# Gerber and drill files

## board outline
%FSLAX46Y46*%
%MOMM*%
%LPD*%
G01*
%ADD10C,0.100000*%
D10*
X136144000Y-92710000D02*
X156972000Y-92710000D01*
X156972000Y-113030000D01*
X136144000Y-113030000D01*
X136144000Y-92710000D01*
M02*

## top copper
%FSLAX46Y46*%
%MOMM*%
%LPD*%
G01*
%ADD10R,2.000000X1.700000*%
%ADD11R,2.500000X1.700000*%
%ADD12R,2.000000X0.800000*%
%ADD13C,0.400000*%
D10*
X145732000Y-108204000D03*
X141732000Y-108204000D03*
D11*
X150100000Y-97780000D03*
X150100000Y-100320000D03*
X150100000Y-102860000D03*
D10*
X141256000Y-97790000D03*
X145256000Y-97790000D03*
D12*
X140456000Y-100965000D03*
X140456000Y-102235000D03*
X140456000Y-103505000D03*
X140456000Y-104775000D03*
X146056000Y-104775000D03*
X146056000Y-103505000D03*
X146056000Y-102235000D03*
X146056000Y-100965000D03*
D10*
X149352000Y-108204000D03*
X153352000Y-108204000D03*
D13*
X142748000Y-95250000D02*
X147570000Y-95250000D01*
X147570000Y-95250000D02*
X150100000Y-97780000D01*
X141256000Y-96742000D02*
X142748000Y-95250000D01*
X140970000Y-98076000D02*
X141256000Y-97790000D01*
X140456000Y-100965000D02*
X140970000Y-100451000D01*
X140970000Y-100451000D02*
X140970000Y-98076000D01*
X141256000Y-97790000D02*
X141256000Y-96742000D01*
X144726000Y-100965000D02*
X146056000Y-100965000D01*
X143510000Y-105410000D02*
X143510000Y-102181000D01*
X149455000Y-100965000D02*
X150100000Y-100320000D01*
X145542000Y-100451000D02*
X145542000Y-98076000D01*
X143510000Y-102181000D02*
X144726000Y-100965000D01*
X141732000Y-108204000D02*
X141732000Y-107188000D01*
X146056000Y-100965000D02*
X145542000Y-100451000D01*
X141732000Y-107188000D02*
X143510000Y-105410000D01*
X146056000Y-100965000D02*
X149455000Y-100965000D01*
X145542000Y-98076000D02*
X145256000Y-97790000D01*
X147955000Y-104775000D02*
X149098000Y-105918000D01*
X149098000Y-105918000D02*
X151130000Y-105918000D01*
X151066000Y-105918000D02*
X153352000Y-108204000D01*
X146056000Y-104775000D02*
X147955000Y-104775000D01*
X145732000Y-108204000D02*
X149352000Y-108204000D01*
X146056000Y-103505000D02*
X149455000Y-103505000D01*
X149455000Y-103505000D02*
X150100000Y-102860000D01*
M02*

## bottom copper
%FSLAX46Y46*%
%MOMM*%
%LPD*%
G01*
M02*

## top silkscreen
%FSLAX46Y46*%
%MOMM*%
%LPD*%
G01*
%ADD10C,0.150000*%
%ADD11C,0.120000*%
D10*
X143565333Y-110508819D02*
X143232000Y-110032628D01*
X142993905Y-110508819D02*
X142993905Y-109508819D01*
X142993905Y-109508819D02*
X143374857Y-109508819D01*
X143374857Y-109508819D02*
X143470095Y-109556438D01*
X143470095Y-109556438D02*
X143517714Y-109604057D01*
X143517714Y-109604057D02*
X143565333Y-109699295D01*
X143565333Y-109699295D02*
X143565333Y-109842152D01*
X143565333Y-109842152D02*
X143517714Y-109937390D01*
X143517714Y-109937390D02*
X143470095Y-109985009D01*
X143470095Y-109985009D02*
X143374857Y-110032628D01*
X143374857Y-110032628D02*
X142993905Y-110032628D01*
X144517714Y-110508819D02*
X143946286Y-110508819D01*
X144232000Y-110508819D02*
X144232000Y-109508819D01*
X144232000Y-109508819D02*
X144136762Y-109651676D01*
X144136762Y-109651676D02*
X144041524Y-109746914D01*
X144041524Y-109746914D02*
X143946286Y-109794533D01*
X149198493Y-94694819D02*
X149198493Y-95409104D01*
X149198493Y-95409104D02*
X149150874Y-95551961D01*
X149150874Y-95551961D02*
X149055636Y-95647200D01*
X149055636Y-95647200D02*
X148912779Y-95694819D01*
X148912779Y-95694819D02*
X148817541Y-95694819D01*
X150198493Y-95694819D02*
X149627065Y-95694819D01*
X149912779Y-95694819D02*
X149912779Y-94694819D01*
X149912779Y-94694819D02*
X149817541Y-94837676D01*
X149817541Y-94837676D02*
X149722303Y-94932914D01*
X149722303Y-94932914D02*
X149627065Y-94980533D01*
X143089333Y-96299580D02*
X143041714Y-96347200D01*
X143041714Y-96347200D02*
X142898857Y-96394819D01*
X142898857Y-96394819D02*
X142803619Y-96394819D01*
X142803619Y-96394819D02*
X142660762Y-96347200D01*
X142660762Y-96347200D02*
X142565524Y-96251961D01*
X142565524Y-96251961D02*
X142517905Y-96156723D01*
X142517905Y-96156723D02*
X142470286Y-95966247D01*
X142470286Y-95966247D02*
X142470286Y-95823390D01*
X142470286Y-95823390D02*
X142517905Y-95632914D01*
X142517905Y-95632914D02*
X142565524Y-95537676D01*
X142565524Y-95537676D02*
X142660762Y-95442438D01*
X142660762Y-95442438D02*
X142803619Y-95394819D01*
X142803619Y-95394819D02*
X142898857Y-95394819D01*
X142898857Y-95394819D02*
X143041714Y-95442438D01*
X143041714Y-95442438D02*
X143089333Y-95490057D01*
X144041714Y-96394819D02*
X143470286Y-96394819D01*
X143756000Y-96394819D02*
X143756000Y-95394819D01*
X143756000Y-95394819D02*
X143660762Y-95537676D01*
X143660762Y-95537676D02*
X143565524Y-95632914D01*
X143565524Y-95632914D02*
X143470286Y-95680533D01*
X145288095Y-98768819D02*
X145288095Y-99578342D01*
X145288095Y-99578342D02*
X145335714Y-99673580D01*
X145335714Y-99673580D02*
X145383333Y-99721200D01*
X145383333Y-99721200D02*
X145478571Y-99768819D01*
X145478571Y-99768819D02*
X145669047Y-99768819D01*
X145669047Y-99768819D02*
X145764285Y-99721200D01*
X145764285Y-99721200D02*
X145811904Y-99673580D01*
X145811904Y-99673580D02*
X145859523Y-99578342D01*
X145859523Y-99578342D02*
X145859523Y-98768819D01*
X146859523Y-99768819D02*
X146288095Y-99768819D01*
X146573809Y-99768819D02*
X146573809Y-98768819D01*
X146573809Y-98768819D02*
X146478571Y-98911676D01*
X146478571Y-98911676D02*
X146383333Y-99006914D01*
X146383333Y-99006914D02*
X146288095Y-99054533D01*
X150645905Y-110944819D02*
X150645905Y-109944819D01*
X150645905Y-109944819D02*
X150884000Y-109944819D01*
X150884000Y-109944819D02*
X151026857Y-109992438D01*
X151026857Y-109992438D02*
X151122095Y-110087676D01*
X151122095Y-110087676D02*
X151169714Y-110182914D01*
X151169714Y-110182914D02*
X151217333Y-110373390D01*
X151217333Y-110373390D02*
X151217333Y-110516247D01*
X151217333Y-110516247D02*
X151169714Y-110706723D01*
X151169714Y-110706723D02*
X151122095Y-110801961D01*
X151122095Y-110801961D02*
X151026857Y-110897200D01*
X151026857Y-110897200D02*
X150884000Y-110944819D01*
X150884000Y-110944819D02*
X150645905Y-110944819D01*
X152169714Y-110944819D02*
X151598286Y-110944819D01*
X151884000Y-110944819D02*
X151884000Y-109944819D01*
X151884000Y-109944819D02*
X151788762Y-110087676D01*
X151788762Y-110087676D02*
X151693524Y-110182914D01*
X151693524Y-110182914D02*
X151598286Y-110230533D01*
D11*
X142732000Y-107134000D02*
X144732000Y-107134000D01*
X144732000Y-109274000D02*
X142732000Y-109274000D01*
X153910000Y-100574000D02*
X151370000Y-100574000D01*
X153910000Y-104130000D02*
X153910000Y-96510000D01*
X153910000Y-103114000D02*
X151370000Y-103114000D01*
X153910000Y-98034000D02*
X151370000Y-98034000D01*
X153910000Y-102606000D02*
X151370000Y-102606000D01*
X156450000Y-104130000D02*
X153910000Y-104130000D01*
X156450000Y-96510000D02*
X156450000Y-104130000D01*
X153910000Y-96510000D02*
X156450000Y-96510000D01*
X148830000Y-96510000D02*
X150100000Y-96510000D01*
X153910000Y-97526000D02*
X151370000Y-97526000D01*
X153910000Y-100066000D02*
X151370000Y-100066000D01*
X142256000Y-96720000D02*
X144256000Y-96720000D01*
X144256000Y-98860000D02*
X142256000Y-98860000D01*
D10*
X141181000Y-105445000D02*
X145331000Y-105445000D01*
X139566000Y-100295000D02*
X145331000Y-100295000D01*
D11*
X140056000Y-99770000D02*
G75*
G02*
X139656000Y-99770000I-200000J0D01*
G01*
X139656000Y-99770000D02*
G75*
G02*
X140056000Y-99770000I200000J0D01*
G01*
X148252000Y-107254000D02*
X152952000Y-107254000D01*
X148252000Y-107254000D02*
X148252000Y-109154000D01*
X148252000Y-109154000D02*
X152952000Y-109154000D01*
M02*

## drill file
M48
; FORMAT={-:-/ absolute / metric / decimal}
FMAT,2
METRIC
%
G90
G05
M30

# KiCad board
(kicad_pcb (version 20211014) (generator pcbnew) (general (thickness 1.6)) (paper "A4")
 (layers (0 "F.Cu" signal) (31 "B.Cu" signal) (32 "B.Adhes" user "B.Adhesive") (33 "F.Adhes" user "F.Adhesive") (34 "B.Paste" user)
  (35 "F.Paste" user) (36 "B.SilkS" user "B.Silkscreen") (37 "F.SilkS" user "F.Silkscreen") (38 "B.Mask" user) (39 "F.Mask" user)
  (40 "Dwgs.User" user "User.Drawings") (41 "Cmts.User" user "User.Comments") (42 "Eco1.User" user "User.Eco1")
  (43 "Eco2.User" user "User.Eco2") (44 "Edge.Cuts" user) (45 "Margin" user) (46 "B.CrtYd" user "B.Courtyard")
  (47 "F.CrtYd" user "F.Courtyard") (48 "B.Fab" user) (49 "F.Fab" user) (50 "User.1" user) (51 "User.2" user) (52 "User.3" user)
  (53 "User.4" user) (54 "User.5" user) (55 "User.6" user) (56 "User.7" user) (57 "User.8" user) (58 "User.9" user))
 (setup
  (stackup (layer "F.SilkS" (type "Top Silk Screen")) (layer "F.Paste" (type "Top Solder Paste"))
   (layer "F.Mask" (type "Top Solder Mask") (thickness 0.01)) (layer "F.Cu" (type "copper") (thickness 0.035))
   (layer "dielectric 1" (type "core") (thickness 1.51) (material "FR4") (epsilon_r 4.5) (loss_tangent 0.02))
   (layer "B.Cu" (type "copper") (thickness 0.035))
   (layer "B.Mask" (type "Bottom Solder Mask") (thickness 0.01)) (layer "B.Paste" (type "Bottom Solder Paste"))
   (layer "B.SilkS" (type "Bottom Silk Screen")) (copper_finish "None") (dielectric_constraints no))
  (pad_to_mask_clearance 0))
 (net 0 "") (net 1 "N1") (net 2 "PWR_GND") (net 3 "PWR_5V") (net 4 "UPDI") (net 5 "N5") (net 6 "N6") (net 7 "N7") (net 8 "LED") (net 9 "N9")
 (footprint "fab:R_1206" (layer "F.Cu") (at 143.732 108.204 180)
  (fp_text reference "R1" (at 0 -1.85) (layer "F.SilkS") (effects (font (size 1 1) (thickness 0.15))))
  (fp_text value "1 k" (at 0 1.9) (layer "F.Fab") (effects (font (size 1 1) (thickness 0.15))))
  (fp_line (start 1 1.07) (end -1 1.07) (layer "F.SilkS") (width 0.12))
  (fp_line (start -1 -1.07) (end 1 -1.07) (layer "F.SilkS") (width 0.12))
  (pad "1" smd rect locked (at -2 0 180) (size 2 1.7) (layers "F.Cu" "F.Paste" "F.Mask") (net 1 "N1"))
  (pad "2" smd rect locked (at 2 0 180) (size 2 1.7) (layers "F.Cu" "F.Paste" "F.Mask") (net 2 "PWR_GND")))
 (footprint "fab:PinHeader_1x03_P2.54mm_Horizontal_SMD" (layer "F.Cu") (at 150.1 97.78)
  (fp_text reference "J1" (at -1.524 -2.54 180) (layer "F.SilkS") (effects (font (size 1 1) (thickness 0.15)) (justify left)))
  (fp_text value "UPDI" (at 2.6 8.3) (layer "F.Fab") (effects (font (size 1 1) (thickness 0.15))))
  (fp_line (start 3.81 2.794) (end 1.27 2.794) (layer "F.SilkS") (width 0.12))
  (fp_line (start 3.81 6.35) (end 3.81 -1.27) (layer "F.SilkS") (width 0.12))
  (fp_line (start 3.81 5.334) (end 1.27 5.334) (layer "F.SilkS") (width 0.12))
  (fp_line (start 3.81 0.254) (end 1.27 0.254) (layer "F.SilkS") (width 0.12))
  (fp_line (start 3.81 4.826) (end 1.27 4.826) (layer "F.SilkS") (width 0.12))
  (fp_line (start 6.35 6.35) (end 3.81 6.35) (layer "F.SilkS") (width 0.12))
  (fp_line (start 6.35 -1.27) (end 6.35 6.35) (layer "F.SilkS") (width 0.12))
  (fp_line (start 3.81 -1.27) (end 6.35 -1.27) (layer "F.SilkS") (width 0.12))
  (fp_line (start -1.27 -1.27) (end 0 -1.27) (layer "F.SilkS") (width 0.12))
  (fp_line (start 3.81 -0.254) (end 1.27 -0.254) (layer "F.SilkS") (width 0.12))
  (fp_line (start 3.81 2.286) (end 1.27 2.286) (layer "F.SilkS") (width 0.12))
  (pad "1" smd rect locked (at 0 0) (size 2.5 1.7) (layers "F.Cu" "F.Paste" "F.Mask") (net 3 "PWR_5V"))
  (pad "2" smd rect locked (at 0 2.54) (size 2.5 1.7) (layers "F.Cu" "F.Paste" "F.Mask") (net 2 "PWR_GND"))
  (pad "3" smd rect locked (at 0 5.08) (size 2.5 1.7) (layers "F.Cu" "F.Paste" "F.Mask") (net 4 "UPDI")))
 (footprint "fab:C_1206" (layer "F.Cu") (at 143.256 97.79)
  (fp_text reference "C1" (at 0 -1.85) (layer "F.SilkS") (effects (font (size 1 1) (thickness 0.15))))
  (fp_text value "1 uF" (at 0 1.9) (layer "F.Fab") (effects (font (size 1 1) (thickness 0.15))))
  (fp_line (start -1 -1.07) (end 1 -1.07) (layer "F.SilkS") (width 0.12))
  (fp_line (start 1 1.07) (end -1 1.07) (layer "F.SilkS") (width 0.12))
  (pad "1" smd rect (at -2 0) (size 2 1.7) (layers "F.Cu" "F.Paste" "F.Mask") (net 3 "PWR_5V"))
  (pad "2" smd rect (at 2 0) (size 2 1.7) (layers "F.Cu" "F.Paste" "F.Mask") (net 2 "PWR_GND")))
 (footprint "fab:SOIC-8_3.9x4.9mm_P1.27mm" (layer "F.Cu") (at 143.256 102.87)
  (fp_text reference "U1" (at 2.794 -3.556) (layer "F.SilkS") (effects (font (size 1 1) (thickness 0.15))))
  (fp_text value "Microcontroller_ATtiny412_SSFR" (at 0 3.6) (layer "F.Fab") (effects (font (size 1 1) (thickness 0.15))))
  (fp_line (start -2.075 2.575) (end 2.075 2.575) (layer "F.SilkS") (width 0.15))
  (fp_line (start -3.69 -2.575) (end 2.075 -2.575) (layer "F.SilkS") (width 0.15))
  (fp_circle (center -3.4 -3.1) (end -3.2 -3.1) (layer "F.SilkS") (width 0.12) (fill none))
  (pad "1" smd rect (at -2.8 -1.905) (size 2 0.8) (layers "F.Cu" "F.Paste" "F.Mask") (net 3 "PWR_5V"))
  (pad "2" smd rect (at -2.8 -0.635) (size 2 0.8) (layers "F.Cu" "F.Paste" "F.Mask") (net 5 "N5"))
  (pad "3" smd rect (at -2.8 0.635) (size 2 0.8) (layers "F.Cu" "F.Paste" "F.Mask") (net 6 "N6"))
  (pad "4" smd rect (at -2.8 1.905) (size 2 0.8) (layers "F.Cu" "F.Paste" "F.Mask") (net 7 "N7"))
  (pad "5" smd rect (at 2.8 1.905) (size 2 0.8) (layers "F.Cu" "F.Paste" "F.Mask") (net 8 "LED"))
  (pad "6" smd rect (at 2.8 0.635) (size 2 0.8) (layers "F.Cu" "F.Paste" "F.Mask") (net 4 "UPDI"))
  (pad "7" smd rect (at 2.8 -0.635) (size 2 0.8) (layers "F.Cu" "F.Paste" "F.Mask") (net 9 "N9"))
  (pad "8" smd rect (at 2.8 -1.905) (size 2 0.8) (layers "F.Cu" "F.Paste" "F.Mask") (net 2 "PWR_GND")))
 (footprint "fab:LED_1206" (layer "F.Cu") (at 151.352 108.204)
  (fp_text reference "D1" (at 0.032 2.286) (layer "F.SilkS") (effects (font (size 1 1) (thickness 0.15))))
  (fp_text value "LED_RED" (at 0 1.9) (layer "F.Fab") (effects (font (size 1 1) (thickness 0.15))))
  (fp_line (start -3.1 -0.95) (end 1.6 -0.95) (layer "F.SilkS") (width 0.12))
  (fp_line (start -3.1 -0.95) (end -3.1 0.95) (layer "F.SilkS") (width 0.12))
  (fp_line (start -3.1 0.95) (end 1.6 0.95) (layer "F.SilkS") (width 0.12))
  (pad "1" smd rect locked (at -2 0) (size 2 1.7) (layers "F.Cu" "F.Paste" "F.Mask") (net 1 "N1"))
  (pad "2" smd rect locked (at 2 0) (size 2 1.7) (layers "F.Cu" "F.Paste" "F.Mask") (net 8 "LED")))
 (gr_rect (start 136.144 92.71) (end 156.972 113.03) (layer "Edge.Cuts") (width 0.1) (fill none))
 (segment (start 142.748 95.25) (end 147.57 95.25) (width 0.4) (layer "F.Cu") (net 3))
 (segment (start 147.57 95.25) (end 150.1 97.78) (width 0.4) (layer "F.Cu") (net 3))
 (segment (start 141.256 96.742) (end 142.748 95.25) (width 0.4) (layer "F.Cu") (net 3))
 (segment (start 140.97 98.076) (end 141.256 97.79) (width 0.4) (layer "F.Cu") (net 3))
 (segment (start 140.456 100.965) (end 140.97 100.451) (width 0.4) (layer "F.Cu") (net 3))
 (segment (start 140.97 100.451) (end 140.97 98.076) (width 0.4) (layer "F.Cu") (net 3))
 (segment (start 141.256 97.79) (end 141.256 96.742) (width 0.4) (layer "F.Cu") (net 3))
 (segment (start 144.726 100.965) (end 146.056 100.965) (width 0.4) (layer "F.Cu") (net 2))
 (segment (start 143.51 105.41) (end 143.51 102.181) (width 0.4) (layer "F.Cu") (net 2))
 (segment (start 149.455 100.965) (end 150.1 100.32) (width 0.4) (layer "F.Cu") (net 2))
 (segment (start 145.542 100.451) (end 145.542 98.076) (width 0.4) (layer "F.Cu") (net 2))
 (segment (start 143.51 102.181) (end 144.726 100.965) (width 0.4) (layer "F.Cu") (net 2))
 (segment (start 141.732 108.204) (end 141.732 107.188) (width 0.4) (layer "F.Cu") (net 2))
 (segment (start 146.056 100.965) (end 145.542 100.451) (width 0.4) (layer "F.Cu") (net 2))
 (segment (start 141.732 107.188) (end 143.51 105.41) (width 0.4) (layer "F.Cu") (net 2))
 (segment (start 146.056 100.965) (end 149.455 100.965) (width 0.4) (layer "F.Cu") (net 2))
 (segment (start 145.542 98.076) (end 145.256 97.79) (width 0.4) (layer "F.Cu") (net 2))
 (segment (start 147.955 104.775) (end 149.098 105.918) (width 0.4) (layer "F.Cu") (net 8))
 (segment (start 149.098 105.918) (end 151.13 105.918) (width 0.4) (layer "F.Cu") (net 8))
 (segment (start 151.066 105.918) (end 153.352 108.204) (width 0.4) (layer "F.Cu") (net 8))
 (segment (start 146.056 104.775) (end 147.955 104.775) (width 0.4) (layer "F.Cu") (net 8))
 (segment (start 145.732 108.204) (end 149.352 108.204) (width 0.4) (layer "F.Cu") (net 1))
 (segment (start 146.056 103.505) (end 149.455 103.505) (width 0.4) (layer "F.Cu") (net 4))
 (segment (start 149.455 103.505) (end 150.1 102.86) (width 0.4) (layer "F.Cu") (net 4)))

